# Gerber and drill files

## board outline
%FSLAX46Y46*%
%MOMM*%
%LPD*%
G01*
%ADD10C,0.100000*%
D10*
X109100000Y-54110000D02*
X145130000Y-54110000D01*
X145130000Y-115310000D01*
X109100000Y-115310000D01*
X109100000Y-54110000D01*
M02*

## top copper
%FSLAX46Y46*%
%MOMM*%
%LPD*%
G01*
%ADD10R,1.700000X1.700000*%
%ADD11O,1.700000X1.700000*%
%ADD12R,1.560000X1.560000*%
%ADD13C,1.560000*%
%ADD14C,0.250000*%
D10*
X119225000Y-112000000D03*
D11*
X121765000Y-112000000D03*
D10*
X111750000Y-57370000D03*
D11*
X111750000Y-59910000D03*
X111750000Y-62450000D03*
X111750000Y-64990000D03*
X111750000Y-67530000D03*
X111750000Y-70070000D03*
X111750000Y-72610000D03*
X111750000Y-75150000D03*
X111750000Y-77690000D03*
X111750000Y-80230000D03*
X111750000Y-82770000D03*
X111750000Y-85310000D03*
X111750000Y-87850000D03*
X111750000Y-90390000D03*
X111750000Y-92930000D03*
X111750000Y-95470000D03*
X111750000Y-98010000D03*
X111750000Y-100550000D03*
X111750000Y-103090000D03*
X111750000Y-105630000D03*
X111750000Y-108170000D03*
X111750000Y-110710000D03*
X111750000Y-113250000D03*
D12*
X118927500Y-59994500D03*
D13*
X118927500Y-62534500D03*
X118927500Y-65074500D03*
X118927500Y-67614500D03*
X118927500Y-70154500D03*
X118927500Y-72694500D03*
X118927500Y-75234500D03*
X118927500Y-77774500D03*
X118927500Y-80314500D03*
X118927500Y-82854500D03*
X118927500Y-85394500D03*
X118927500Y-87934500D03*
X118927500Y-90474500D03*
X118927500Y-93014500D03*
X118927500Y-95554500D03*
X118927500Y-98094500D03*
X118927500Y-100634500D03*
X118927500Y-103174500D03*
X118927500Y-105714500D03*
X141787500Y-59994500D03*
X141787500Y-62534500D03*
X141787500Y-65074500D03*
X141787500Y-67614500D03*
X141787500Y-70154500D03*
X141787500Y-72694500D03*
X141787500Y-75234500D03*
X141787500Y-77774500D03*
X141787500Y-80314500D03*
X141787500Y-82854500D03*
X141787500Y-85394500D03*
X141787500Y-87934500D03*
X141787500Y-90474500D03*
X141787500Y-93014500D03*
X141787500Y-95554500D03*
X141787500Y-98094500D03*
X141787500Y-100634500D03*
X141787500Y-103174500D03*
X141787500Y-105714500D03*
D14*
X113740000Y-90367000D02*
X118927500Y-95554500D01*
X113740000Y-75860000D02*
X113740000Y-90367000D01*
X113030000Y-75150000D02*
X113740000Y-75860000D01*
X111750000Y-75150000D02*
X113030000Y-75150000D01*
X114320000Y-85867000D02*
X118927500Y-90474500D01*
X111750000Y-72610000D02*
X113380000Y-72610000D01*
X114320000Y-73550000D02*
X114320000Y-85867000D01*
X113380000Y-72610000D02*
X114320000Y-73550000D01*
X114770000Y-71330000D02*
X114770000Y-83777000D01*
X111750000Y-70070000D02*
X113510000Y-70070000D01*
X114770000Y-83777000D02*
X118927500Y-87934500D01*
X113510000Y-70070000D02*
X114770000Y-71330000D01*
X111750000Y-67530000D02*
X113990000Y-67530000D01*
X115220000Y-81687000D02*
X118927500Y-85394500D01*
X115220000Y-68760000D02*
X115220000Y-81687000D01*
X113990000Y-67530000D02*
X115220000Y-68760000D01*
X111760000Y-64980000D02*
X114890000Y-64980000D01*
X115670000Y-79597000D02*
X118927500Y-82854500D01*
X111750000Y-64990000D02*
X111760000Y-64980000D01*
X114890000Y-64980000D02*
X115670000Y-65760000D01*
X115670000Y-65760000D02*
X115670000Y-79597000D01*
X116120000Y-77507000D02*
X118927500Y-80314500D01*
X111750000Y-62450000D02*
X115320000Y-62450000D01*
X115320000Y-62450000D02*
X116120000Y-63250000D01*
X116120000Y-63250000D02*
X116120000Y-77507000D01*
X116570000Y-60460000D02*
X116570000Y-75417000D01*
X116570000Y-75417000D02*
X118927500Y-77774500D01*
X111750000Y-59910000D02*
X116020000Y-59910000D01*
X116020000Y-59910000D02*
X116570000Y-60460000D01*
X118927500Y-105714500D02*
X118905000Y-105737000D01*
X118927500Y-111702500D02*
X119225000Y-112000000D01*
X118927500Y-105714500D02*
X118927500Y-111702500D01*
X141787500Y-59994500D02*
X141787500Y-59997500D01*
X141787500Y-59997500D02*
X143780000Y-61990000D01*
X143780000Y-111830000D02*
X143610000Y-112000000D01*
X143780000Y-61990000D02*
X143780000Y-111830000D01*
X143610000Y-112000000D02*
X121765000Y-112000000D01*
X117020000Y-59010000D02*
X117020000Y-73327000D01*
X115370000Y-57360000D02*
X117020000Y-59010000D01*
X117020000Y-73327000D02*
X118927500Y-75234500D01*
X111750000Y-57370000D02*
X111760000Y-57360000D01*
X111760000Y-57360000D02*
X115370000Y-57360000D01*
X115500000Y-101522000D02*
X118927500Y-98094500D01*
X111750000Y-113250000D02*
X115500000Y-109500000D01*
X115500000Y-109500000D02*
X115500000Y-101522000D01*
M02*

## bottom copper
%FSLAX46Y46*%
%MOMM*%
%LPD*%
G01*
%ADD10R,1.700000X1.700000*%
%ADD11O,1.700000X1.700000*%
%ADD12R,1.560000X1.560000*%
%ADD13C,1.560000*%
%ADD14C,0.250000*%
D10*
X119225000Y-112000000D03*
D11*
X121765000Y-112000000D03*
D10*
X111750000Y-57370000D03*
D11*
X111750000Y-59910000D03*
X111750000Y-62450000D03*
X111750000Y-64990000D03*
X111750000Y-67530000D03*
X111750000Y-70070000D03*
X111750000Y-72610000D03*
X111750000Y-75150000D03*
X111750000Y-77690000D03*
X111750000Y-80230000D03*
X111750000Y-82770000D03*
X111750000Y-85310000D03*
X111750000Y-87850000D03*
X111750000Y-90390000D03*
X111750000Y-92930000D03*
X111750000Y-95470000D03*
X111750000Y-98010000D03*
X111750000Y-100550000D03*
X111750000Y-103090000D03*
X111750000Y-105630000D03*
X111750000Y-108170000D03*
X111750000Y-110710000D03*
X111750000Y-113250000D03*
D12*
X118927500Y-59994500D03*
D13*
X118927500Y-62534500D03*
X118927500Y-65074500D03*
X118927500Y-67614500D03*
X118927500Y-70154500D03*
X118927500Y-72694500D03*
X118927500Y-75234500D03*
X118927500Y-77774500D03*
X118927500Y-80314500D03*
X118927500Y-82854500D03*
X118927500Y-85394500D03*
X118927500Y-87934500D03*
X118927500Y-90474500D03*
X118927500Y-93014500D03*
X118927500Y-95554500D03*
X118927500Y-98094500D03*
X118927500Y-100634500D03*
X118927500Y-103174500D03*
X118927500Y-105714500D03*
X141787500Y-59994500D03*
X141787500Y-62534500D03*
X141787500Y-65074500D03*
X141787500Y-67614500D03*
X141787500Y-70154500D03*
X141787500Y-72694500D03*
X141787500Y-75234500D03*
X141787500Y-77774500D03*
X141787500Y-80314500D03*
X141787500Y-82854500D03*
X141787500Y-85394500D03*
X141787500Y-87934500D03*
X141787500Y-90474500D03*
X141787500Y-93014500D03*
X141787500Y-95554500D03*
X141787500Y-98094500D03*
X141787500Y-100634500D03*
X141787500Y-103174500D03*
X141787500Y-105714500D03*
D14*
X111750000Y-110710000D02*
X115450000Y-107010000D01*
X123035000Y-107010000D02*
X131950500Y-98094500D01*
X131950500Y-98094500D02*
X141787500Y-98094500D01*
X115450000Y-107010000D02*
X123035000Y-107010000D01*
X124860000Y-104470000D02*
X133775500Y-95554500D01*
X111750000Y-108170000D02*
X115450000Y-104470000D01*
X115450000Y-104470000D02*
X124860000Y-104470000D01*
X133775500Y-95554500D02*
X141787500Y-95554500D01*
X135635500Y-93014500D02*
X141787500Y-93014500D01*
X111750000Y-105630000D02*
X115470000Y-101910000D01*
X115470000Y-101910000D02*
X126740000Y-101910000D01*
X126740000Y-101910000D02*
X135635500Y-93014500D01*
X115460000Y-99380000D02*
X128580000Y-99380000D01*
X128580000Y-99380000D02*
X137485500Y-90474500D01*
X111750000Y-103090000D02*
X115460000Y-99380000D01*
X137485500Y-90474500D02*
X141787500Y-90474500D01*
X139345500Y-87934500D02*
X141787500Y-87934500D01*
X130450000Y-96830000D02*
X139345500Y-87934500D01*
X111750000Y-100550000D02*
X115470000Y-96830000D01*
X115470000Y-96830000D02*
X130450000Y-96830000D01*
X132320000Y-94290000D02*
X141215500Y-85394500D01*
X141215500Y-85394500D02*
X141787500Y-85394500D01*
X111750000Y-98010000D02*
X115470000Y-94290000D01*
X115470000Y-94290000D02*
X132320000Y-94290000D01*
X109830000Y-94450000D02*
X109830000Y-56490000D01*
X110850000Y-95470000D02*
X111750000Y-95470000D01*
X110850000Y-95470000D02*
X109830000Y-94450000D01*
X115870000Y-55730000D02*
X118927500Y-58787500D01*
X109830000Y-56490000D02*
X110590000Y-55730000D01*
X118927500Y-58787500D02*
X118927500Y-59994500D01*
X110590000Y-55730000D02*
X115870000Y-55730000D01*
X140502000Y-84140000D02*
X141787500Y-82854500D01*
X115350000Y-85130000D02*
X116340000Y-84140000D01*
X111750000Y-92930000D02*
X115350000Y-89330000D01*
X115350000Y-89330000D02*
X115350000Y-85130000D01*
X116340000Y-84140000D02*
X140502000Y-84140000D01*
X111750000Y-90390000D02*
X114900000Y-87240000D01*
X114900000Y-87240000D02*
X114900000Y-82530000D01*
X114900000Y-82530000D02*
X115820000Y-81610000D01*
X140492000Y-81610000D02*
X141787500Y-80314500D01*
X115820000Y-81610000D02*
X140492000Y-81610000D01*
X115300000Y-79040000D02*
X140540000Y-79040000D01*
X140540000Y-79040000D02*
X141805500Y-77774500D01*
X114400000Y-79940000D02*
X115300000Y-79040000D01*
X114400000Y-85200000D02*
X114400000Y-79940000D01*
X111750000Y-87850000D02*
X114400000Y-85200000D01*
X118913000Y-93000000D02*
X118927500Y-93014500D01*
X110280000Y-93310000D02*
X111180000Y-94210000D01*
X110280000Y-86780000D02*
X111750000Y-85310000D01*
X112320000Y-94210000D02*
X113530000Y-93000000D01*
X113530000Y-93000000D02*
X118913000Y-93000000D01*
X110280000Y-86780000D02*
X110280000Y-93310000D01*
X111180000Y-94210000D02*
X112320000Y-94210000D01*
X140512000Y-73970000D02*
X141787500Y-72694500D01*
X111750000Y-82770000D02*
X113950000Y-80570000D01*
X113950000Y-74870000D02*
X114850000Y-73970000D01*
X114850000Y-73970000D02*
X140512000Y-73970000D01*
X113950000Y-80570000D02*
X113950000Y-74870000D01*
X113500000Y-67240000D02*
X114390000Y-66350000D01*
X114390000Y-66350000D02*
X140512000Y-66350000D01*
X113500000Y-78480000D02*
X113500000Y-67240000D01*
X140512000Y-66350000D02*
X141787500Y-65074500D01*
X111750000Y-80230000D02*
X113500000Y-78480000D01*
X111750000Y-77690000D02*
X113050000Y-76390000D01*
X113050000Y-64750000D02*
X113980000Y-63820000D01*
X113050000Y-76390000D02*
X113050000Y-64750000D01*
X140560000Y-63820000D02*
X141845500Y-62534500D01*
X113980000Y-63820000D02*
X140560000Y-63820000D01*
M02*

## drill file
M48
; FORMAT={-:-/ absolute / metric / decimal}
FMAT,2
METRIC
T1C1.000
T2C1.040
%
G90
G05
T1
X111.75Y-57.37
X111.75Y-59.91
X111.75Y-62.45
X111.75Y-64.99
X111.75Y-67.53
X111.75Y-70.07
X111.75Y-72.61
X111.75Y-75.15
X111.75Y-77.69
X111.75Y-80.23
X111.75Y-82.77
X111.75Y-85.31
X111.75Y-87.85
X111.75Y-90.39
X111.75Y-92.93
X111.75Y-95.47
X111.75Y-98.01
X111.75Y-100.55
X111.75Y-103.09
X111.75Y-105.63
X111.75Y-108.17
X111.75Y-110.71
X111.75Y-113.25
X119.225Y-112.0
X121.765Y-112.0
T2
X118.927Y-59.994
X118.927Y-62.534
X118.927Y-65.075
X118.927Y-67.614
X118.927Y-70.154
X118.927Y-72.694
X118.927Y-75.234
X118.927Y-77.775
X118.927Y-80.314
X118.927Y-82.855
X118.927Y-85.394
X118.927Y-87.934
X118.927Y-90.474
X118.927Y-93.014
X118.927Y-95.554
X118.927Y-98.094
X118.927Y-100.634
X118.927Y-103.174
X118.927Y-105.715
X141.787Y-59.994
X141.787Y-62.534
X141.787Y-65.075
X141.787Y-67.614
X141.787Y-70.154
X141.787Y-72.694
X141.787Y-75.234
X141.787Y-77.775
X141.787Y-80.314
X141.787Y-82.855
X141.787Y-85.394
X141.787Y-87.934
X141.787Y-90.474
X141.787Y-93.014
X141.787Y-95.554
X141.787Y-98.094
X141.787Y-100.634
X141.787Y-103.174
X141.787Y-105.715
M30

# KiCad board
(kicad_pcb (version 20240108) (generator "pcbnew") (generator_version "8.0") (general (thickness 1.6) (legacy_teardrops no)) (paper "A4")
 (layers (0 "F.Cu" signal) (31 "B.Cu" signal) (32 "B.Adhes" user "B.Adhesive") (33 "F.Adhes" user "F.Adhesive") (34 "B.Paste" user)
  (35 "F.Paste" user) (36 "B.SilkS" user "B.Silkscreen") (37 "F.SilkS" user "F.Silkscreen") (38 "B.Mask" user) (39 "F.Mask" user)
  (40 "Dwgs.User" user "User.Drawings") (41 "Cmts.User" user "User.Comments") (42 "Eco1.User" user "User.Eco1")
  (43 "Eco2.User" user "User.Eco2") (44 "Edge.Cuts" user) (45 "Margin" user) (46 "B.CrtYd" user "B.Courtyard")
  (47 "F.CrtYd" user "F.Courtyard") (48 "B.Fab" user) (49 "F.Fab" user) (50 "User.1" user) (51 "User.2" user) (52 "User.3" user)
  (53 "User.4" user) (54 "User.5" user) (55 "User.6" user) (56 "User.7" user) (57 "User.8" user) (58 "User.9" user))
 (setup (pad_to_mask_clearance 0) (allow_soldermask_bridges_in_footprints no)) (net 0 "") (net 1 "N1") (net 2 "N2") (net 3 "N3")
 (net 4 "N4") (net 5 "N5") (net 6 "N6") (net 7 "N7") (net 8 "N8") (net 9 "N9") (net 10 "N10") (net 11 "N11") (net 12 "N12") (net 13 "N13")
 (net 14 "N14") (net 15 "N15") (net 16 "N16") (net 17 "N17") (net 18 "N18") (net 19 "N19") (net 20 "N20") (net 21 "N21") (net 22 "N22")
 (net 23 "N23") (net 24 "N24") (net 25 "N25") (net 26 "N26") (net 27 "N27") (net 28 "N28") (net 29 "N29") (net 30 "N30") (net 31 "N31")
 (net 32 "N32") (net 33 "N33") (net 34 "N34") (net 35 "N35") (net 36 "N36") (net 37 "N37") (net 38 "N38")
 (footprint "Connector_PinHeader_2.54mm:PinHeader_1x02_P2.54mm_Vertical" (layer "F.Cu") (at 119.225 112 90)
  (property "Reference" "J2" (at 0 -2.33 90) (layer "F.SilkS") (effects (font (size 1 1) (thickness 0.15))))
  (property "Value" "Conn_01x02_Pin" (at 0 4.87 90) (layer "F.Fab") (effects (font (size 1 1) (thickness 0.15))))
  (pad "1" thru_hole rect (at 0 0 90) (size 1.7 1.7) (drill 1) (layers "*.Cu" "*.Mask") (remove_unused_layers no) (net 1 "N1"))
  (pad "2" thru_hole oval (at 0 2.54 90) (size 1.7 1.7) (drill 1) (layers "*.Cu" "*.Mask") (remove_unused_layers no) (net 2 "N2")))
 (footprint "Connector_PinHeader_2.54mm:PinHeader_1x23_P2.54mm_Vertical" (layer "F.Cu") (at 111.75 57.37)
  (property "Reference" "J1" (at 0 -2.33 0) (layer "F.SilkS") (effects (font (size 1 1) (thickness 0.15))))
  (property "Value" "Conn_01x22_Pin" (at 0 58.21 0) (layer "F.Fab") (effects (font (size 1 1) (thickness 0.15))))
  (pad "1" thru_hole rect (at 0 0) (size 1.7 1.7) (drill 1) (layers "*.Cu" "*.Mask") (remove_unused_layers no) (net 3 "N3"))
  (pad "2" thru_hole oval (at 0 2.54) (size 1.7 1.7) (drill 1) (layers "*.Cu" "*.Mask") (remove_unused_layers no) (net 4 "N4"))
  (pad "3" thru_hole oval (at 0 5.08) (size 1.7 1.7) (drill 1) (layers "*.Cu" "*.Mask") (remove_unused_layers no) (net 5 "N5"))
  (pad "4" thru_hole oval (at 0 7.62) (size 1.7 1.7) (drill 1) (layers "*.Cu" "*.Mask") (remove_unused_layers no) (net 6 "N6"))
  (pad "5" thru_hole oval (at 0 10.16) (size 1.7 1.7) (drill 1) (layers "*.Cu" "*.Mask") (remove_unused_layers no) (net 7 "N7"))
  (pad "6" thru_hole oval (at 0 12.7) (size 1.7 1.7) (drill 1) (layers "*.Cu" "*.Mask") (remove_unused_layers no) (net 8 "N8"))
  (pad "7" thru_hole oval (at 0 15.24) (size 1.7 1.7) (drill 1) (layers "*.Cu" "*.Mask") (remove_unused_layers no) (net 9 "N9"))
  (pad "8" thru_hole oval (at 0 17.78) (size 1.7 1.7) (drill 1) (layers "*.Cu" "*.Mask") (remove_unused_layers no) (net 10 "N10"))
  (pad "9" thru_hole oval (at 0 20.32) (size 1.7 1.7) (drill 1) (layers "*.Cu" "*.Mask") (remove_unused_layers no) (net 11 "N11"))
  (pad "10" thru_hole oval (at 0 22.86) (size 1.7 1.7) (drill 1) (layers "*.Cu" "*.Mask") (remove_unused_layers no) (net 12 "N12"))
  (pad "11" thru_hole oval (at 0 25.4) (size 1.7 1.7) (drill 1) (layers "*.Cu" "*.Mask") (remove_unused_layers no) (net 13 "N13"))
  (pad "12" thru_hole oval (at 0 27.94) (size 1.7 1.7) (drill 1) (layers "*.Cu" "*.Mask") (remove_unused_layers no) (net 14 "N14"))
  (pad "13" thru_hole oval (at 0 30.48) (size 1.7 1.7) (drill 1) (layers "*.Cu" "*.Mask") (remove_unused_layers no) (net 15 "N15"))
  (pad "14" thru_hole oval (at 0 33.02) (size 1.7 1.7) (drill 1) (layers "*.Cu" "*.Mask") (remove_unused_layers no) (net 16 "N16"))
  (pad "15" thru_hole oval (at 0 35.56) (size 1.7 1.7) (drill 1) (layers "*.Cu" "*.Mask") (remove_unused_layers no) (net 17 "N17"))
  (pad "16" thru_hole oval (at 0 38.1) (size 1.7 1.7) (drill 1) (layers "*.Cu" "*.Mask") (remove_unused_layers no) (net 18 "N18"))
  (pad "17" thru_hole oval (at 0 40.64) (size 1.7 1.7) (drill 1) (layers "*.Cu" "*.Mask") (remove_unused_layers no) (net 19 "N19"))
  (pad "18" thru_hole oval (at 0 43.18) (size 1.7 1.7) (drill 1) (layers "*.Cu" "*.Mask") (remove_unused_layers no) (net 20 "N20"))
  (pad "19" thru_hole oval (at 0 45.72) (size 1.7 1.7) (drill 1) (layers "*.Cu" "*.Mask") (remove_unused_layers no) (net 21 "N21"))
  (pad "20" thru_hole oval (at 0 48.26) (size 1.7 1.7) (drill 1) (layers "*.Cu" "*.Mask") (remove_unused_layers no) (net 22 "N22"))
  (pad "21" thru_hole oval (at 0 50.8) (size 1.7 1.7) (drill 1) (layers "*.Cu" "*.Mask") (remove_unused_layers no) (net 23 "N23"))
  (pad "22" thru_hole oval (at 0 53.34) (size 1.7 1.7) (drill 1) (layers "*.Cu" "*.Mask") (remove_unused_layers no) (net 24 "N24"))
  (pad "23" thru_hole oval (at 0 55.88) (size 1.7 1.7) (drill 1) (layers "*.Cu" "*.Mask") (remove_unused_layers no) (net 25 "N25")))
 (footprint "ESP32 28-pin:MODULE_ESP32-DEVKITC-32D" (layer "F.Cu") (at 131.6275 79.7545)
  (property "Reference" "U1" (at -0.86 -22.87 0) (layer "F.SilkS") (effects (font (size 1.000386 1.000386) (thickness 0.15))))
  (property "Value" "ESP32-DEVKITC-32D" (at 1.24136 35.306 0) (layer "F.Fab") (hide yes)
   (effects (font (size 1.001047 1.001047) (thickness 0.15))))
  (pad "J2-1" thru_hole rect (at -12.7 -19.76) (size 1.56 1.56) (drill 1.04) (layers "*.Cu" "*.Mask") (remove_unused_layers no)
   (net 18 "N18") (solder_mask_margin 0.102))
  (pad "J2-2" thru_hole circle (at -12.7 -17.22) (size 1.56 1.56) (drill 1.04) (layers "*.Cu" "*.Mask") (remove_unused_layers no)
   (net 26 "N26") (solder_mask_margin 0.102))
  (pad "J2-3" thru_hole circle (at -12.7 -14.68) (size 1.56 1.56) (drill 1.04) (layers "*.Cu" "*.Mask") (remove_unused_layers no)
   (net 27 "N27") (solder_mask_margin 0.102))
  (pad "J2-4" thru_hole circle (at -12.7 -12.14) (size 1.56 1.56) (drill 1.04) (layers "*.Cu" "*.Mask") (remove_unused_layers no)
   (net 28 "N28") (solder_mask_margin 0.102))
  (pad "J2-5" thru_hole circle (at -12.7 -9.6) (size 1.56 1.56) (drill 1.04) (layers "*.Cu" "*.Mask") (remove_unused_layers no)
   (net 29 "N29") (solder_mask_margin 0.102))
  (pad "J2-6" thru_hole circle (at -12.7 -7.06) (size 1.56 1.56) (drill 1.04) (layers "*.Cu" "*.Mask") (remove_unused_layers no)
   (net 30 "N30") (solder_mask_margin 0.102))
  (pad "J2-7" thru_hole circle (at -12.7 -4.52) (size 1.56 1.56) (drill 1.04) (layers "*.Cu" "*.Mask") (remove_unused_layers no)
   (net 3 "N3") (solder_mask_margin 0.102))
  (pad "J2-8" thru_hole circle (at -12.7 -1.98) (size 1.56 1.56) (drill 1.04) (layers "*.Cu" "*.Mask") (remove_unused_layers no)
   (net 4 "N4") (solder_mask_margin 0.102))
  (pad "J2-9" thru_hole circle (at -12.7 0.56) (size 1.56 1.56) (drill 1.04) (layers "*.Cu" "*.Mask") (remove_unused_layers no) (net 5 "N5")
   (solder_mask_margin 0.102))
  (pad "J2-10" thru_hole circle (at -12.7 3.1) (size 1.56 1.56) (drill 1.04) (layers "*.Cu" "*.Mask") (remove_unused_layers no) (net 6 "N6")
   (solder_mask_margin 0.102))
  (pad "J2-11" thru_hole circle (at -12.7 5.64) (size 1.56 1.56) (drill 1.04) (layers "*.Cu" "*.Mask") (remove_unused_layers no)
   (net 7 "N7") (solder_mask_margin 0.102))
  (pad "J2-12" thru_hole circle (at -12.7 8.18) (size 1.56 1.56) (drill 1.04) (layers "*.Cu" "*.Mask") (remove_unused_layers no)
   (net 8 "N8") (solder_mask_margin 0.102))
  (pad "J2-13" thru_hole circle (at -12.7 10.72) (size 1.56 1.56) (drill 1.04) (layers "*.Cu" "*.Mask") (remove_unused_layers no)
   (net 9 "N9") (solder_mask_margin 0.102))
  (pad "J2-14" thru_hole circle (at -12.7 13.26) (size 1.56 1.56) (drill 1.04) (layers "*.Cu" "*.Mask") (remove_unused_layers no)
   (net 14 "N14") (solder_mask_margin 0.102))
  (pad "J2-15" thru_hole circle (at -12.7 15.8) (size 1.56 1.56) (drill 1.04) (layers "*.Cu" "*.Mask") (remove_unused_layers no)
   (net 10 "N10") (solder_mask_margin 0.102))
  (pad "J2-16" thru_hole circle (at -12.7 18.34) (size 1.56 1.56) (drill 1.04) (layers "*.Cu" "*.Mask") (remove_unused_layers no)
   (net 25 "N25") (solder_mask_margin 0.102))
  (pad "J2-17" thru_hole circle (at -12.7 20.88) (size 1.56 1.56) (drill 1.04) (layers "*.Cu" "*.Mask") (remove_unused_layers no)
   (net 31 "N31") (solder_mask_margin 0.102))
  (pad "J2-18" thru_hole circle (at -12.7 23.42) (size 1.56 1.56) (drill 1.04) (layers "*.Cu" "*.Mask") (remove_unused_layers no)
   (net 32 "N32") (solder_mask_margin 0.102))
  (pad "J2-19" thru_hole circle (at -12.7 25.96) (size 1.56 1.56) (drill 1.04) (layers "*.Cu" "*.Mask") (remove_unused_layers no)
   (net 1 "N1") (solder_mask_margin 0.102))
  (pad "J3-1" thru_hole circle (at 10.16 -19.76) (size 1.56 1.56) (drill 1.04) (layers "*.Cu" "*.Mask") (remove_unused_layers no)
   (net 2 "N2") (solder_mask_margin 0.102))
  (pad "J3-2" thru_hole circle (at 10.16 -17.22) (size 1.56 1.56) (drill 1.04) (layers "*.Cu" "*.Mask") (remove_unused_layers no)
   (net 11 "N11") (solder_mask_margin 0.102))
  (pad "J3-3" thru_hole circle (at 10.16 -14.68) (size 1.56 1.56) (drill 1.04) (layers "*.Cu" "*.Mask") (remove_unused_layers no)
   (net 12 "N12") (solder_mask_margin 0.102))
  (pad "J3-4" thru_hole circle (at 10.16 -12.14) (size 1.56 1.56) (drill 1.04) (layers "*.Cu" "*.Mask") (remove_unused_layers no)
   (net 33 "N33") (solder_mask_margin 0.102))
  (pad "J3-5" thru_hole circle (at 10.16 -9.6) (size 1.56 1.56) (drill 1.04) (layers "*.Cu" "*.Mask") (remove_unused_layers no)
   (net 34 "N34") (solder_mask_margin 0.102))
  (pad "J3-6" thru_hole circle (at 10.16 -7.06) (size 1.56 1.56) (drill 1.04) (layers "*.Cu" "*.Mask") (remove_unused_layers no)
   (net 13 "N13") (solder_mask_margin 0.102))
  (pad "J3-7" thru_hole circle (at 10.16 -4.52) (size 1.56 1.56) (drill 1.04) (layers "*.Cu" "*.Mask") (remove_unused_layers no)
   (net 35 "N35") (solder_mask_margin 0.102))
  (pad "J3-8" thru_hole circle (at 10.16 -1.98) (size 1.56 1.56) (drill 1.04) (layers "*.Cu" "*.Mask") (remove_unused_layers no)
   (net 15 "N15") (solder_mask_margin 0.102))
  (pad "J3-9" thru_hole circle (at 10.16 0.56) (size 1.56 1.56) (drill 1.04) (layers "*.Cu" "*.Mask") (remove_unused_layers no)
   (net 16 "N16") (solder_mask_margin 0.102))
  (pad "J3-10" thru_hole circle (at 10.16 3.1) (size 1.56 1.56) (drill 1.04) (layers "*.Cu" "*.Mask") (remove_unused_layers no)
   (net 17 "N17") (solder_mask_margin 0.102))
  (pad "J3-11" thru_hole circle (at 10.16 5.64) (size 1.56 1.56) (drill 1.04) (layers "*.Cu" "*.Mask") (remove_unused_layers no)
   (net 19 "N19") (solder_mask_margin 0.102))
  (pad "J3-12" thru_hole circle (at 10.16 8.18) (size 1.56 1.56) (drill 1.04) (layers "*.Cu" "*.Mask") (remove_unused_layers no)
   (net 20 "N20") (solder_mask_margin 0.102))
  (pad "J3-13" thru_hole circle (at 10.16 10.72) (size 1.56 1.56) (drill 1.04) (layers "*.Cu" "*.Mask") (remove_unused_layers no)
   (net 21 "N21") (solder_mask_margin 0.102))
  (pad "J3-14" thru_hole circle (at 10.16 13.26) (size 1.56 1.56) (drill 1.04) (layers "*.Cu" "*.Mask") (remove_unused_layers no)
   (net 22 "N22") (solder_mask_margin 0.102))
  (pad "J3-15" thru_hole circle (at 10.16 15.8) (size 1.56 1.56) (drill 1.04) (layers "*.Cu" "*.Mask") (remove_unused_layers no)
   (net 23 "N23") (solder_mask_margin 0.102))
  (pad "J3-16" thru_hole circle (at 10.16 18.34) (size 1.56 1.56) (drill 1.04) (layers "*.Cu" "*.Mask") (remove_unused_layers no)
   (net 24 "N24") (solder_mask_margin 0.102))
  (pad "J3-17" thru_hole circle (at 10.16 20.88) (size 1.56 1.56) (drill 1.04) (layers "*.Cu" "*.Mask") (remove_unused_layers no)
   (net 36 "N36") (solder_mask_margin 0.102))
  (pad "J3-18" thru_hole circle (at 10.16 23.42) (size 1.56 1.56) (drill 1.04) (layers "*.Cu" "*.Mask") (remove_unused_layers no)
   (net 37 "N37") (solder_mask_margin 0.102))
  (pad "J3-19" thru_hole circle (at 10.16 25.96) (size 1.56 1.56) (drill 1.04) (layers "*.Cu" "*.Mask") (remove_unused_layers no)
   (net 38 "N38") (solder_mask_margin 0.102)))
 (gr_rect (start 109.1 54.11) (end 145.13 115.31) (stroke (width 0.1) (type default)) (fill none) (layer "Edge.Cuts"))
 (segment (start 111.75 110.71) (end 115.45 107.01) (width 0.25) (layer "B.Cu") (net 24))
 (segment (start 123.035 107.01) (end 131.9505 98.0945) (width 0.25) (layer "B.Cu") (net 24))
 (segment (start 131.9505 98.0945) (end 141.7875 98.0945) (width 0.25) (layer "B.Cu") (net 24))
 (segment (start 115.45 107.01) (end 123.035 107.01) (width 0.25) (layer "B.Cu") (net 24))
 (segment (start 124.86 104.47) (end 133.7755 95.5545) (width 0.25) (layer "B.Cu") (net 23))
 (segment (start 111.75 108.17) (end 115.45 104.47) (width 0.25) (layer "B.Cu") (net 23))
 (segment (start 115.45 104.47) (end 124.86 104.47) (width 0.25) (layer "B.Cu") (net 23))
 (segment (start 133.7755 95.5545) (end 141.7875 95.5545) (width 0.25) (layer "B.Cu") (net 23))
 (segment (start 135.6355 93.0145) (end 141.7875 93.0145) (width 0.25) (layer "B.Cu") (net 22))
 (segment (start 111.75 105.63) (end 115.47 101.91) (width 0.25) (layer "B.Cu") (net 22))
 (segment (start 115.47 101.91) (end 126.74 101.91) (width 0.25) (layer "B.Cu") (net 22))
 (segment (start 126.74 101.91) (end 135.6355 93.0145) (width 0.25) (layer "B.Cu") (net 22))
 (segment (start 115.46 99.38) (end 128.58 99.38) (width 0.25) (layer "B.Cu") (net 21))
 (segment (start 128.58 99.38) (end 137.4855 90.4745) (width 0.25) (layer "B.Cu") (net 21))
 (segment (start 111.75 103.09) (end 115.46 99.38) (width 0.25) (layer "B.Cu") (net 21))
 (segment (start 137.4855 90.4745) (end 141.7875 90.4745) (width 0.25) (layer "B.Cu") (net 21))
 (segment (start 139.3455 87.9345) (end 141.7875 87.9345) (width 0.25) (layer "B.Cu") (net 20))
 (segment (start 130.45 96.83) (end 139.3455 87.9345) (width 0.25) (layer "B.Cu") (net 20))
 (segment (start 111.75 100.55) (end 115.47 96.83) (width 0.25) (layer "B.Cu") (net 20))
 (segment (start 115.47 96.83) (end 130.45 96.83) (width 0.25) (layer "B.Cu") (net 20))
 (segment (start 132.32 94.29) (end 141.2155 85.3945) (width 0.25) (layer "B.Cu") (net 19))
 (segment (start 141.2155 85.3945) (end 141.7875 85.3945) (width 0.25) (layer "B.Cu") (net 19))
 (segment (start 111.75 98.01) (end 115.47 94.29) (width 0.25) (layer "B.Cu") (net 19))
 (segment (start 115.47 94.29) (end 132.32 94.29) (width 0.25) (layer "B.Cu") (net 19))
 (segment (start 109.83 94.45) (end 109.83 56.49) (width 0.25) (layer "B.Cu") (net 18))
 (segment (start 110.85 95.47) (end 111.75 95.47) (width 0.25) (layer "B.Cu") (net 18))
 (segment (start 110.85 95.47) (end 109.83 94.45) (width 0.25) (layer "B.Cu") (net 18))
 (segment (start 115.87 55.73) (end 118.9275 58.7875) (width 0.25) (layer "B.Cu") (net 18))
 (segment (start 109.83 56.49) (end 110.59 55.73) (width 0.25) (layer "B.Cu") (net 18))
 (segment (start 118.9275 58.7875) (end 118.9275 59.9945) (width 0.25) (layer "B.Cu") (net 18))
 (segment (start 110.59 55.73) (end 115.87 55.73) (width 0.25) (layer "B.Cu") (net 18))
 (segment (start 140.502 84.14) (end 141.7875 82.8545) (width 0.25) (layer "B.Cu") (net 17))
 (segment (start 115.35 85.13) (end 116.34 84.14) (width 0.25) (layer "B.Cu") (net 17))
 (segment (start 111.75 92.93) (end 115.35 89.33) (width 0.25) (layer "B.Cu") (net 17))
 (segment (start 115.35 89.33) (end 115.35 85.13) (width 0.25) (layer "B.Cu") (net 17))
 (segment (start 116.34 84.14) (end 140.502 84.14) (width 0.25) (layer "B.Cu") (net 17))
 (segment (start 111.75 90.39) (end 114.9 87.24) (width 0.25) (layer "B.Cu") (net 16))
 (segment (start 114.9 87.24) (end 114.9 82.53) (width 0.25) (layer "B.Cu") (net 16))
 (segment (start 114.9 82.53) (end 115.82 81.61) (width 0.25) (layer "B.Cu") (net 16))
 (segment (start 140.492 81.61) (end 141.7875 80.3145) (width 0.25) (layer "B.Cu") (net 16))
 (segment (start 115.82 81.61) (end 140.492 81.61) (width 0.25) (layer "B.Cu") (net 16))
 (segment (start 115.3 79.04) (end 140.54 79.04) (width 0.25) (layer "B.Cu") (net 15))
 (segment (start 140.54 79.04) (end 141.8055 77.7745) (width 0.25) (layer "B.Cu") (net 15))
 (segment (start 114.4 79.94) (end 115.3 79.04) (width 0.25) (layer "B.Cu") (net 15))
 (segment (start 114.4 85.2) (end 114.4 79.94) (width 0.25) (layer "B.Cu") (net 15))
 (segment (start 111.75 87.85) (end 114.4 85.2) (width 0.25) (layer "B.Cu") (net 15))
 (segment (start 118.913 93) (end 118.9275 93.0145) (width 0.25) (layer "B.Cu") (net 14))
 (segment (start 110.28 93.31) (end 111.18 94.21) (width 0.25) (layer "B.Cu") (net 14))
 (segment (start 110.28 86.78) (end 111.75 85.31) (width 0.25) (layer "B.Cu") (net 14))
 (segment (start 112.32 94.21) (end 113.53 93) (width 0.25) (layer "B.Cu") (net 14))
 (segment (start 113.53 93) (end 118.913 93) (width 0.25) (layer "B.Cu") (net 14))
 (segment (start 110.28 86.78) (end 110.28 93.31) (width 0.25) (layer "B.Cu") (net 14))
 (segment (start 111.18 94.21) (end 112.32 94.21) (width 0.25) (layer "B.Cu") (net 14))
 (segment (start 140.512 73.97) (end 141.7875 72.6945) (width 0.25) (layer "B.Cu") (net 13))
 (segment (start 111.75 82.77) (end 113.95 80.57) (width 0.25) (layer "B.Cu") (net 13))
 (segment (start 113.95 74.87) (end 114.85 73.97) (width 0.25) (layer "B.Cu") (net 13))
 (segment (start 114.85 73.97) (end 140.512 73.97) (width 0.25) (layer "B.Cu") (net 13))
 (segment (start 113.95 80.57) (end 113.95 74.87) (width 0.25) (layer "B.Cu") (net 13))
 (segment (start 113.5 67.24) (end 114.39 66.35) (width 0.25) (layer "B.Cu") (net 12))
 (segment (start 114.39 66.35) (end 140.512 66.35) (width 0.25) (layer "B.Cu") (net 12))
 (segment (start 113.5 78.48) (end 113.5 67.24) (width 0.25) (layer "B.Cu") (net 12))
 (segment (start 140.512 66.35) (end 141.7875 65.0745) (width 0.25) (layer "B.Cu") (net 12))
 (segment (start 111.75 80.23) (end 113.5 78.48) (width 0.25) (layer "B.Cu") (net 12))
 (segment (start 111.75 77.69) (end 113.05 76.39) (width 0.25) (layer "B.Cu") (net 11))
 (segment (start 113.05 64.75) (end 113.98 63.82) (width 0.25) (layer "B.Cu") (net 11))
 (segment (start 113.05 76.39) (end 113.05 64.75) (width 0.25) (layer "B.Cu") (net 11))
 (segment (start 140.56 63.82) (end 141.8455 62.5345) (width 0.25) (layer "B.Cu") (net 11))
 (segment (start 113.98 63.82) (end 140.56 63.82) (width 0.25) (layer "B.Cu") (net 11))
 (segment (start 113.74 90.367) (end 118.9275 95.5545) (width 0.25) (layer "F.Cu") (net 10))
 (segment (start 113.74 75.86) (end 113.74 90.367) (width 0.25) (layer "F.Cu") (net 10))
 (segment (start 113.03 75.15) (end 113.74 75.86) (width 0.25) (layer "F.Cu") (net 10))
 (segment (start 111.75 75.15) (end 113.03 75.15) (width 0.25) (layer "F.Cu") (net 10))
 (segment (start 114.32 85.867) (end 118.9275 90.4745) (width 0.25) (layer "F.Cu") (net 9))
 (segment (start 111.75 72.61) (end 113.38 72.61) (width 0.25) (layer "F.Cu") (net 9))
 (segment (start 114.32 73.55) (end 114.32 85.867) (width 0.25) (layer "F.Cu") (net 9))
 (segment (start 113.38 72.61) (end 114.32 73.55) (width 0.25) (layer "F.Cu") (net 9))
 (segment (start 114.77 71.33) (end 114.77 83.777) (width 0.25) (layer "F.Cu") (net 8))
 (segment (start 111.75 70.07) (end 113.51 70.07) (width 0.25) (layer "F.Cu") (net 8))
 (segment (start 114.77 83.777) (end 118.9275 87.9345) (width 0.25) (layer "F.Cu") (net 8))
 (segment (start 113.51 70.07) (end 114.77 71.33) (width 0.25) (layer "F.Cu") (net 8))
 (segment (start 111.75 67.53) (end 113.99 67.53) (width 0.25) (layer "F.Cu") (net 7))
 (segment (start 115.22 81.687) (end 118.9275 85.3945) (width 0.25) (layer "F.Cu") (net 7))
 (segment (start 115.22 68.76) (end 115.22 81.687) (width 0.25) (layer "F.Cu") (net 7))
 (segment (start 113.99 67.53) (end 115.22 68.76) (width 0.25) (layer "F.Cu") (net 7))
 (segment (start 111.76 64.98) (end 114.89 64.98) (width 0.25) (layer "F.Cu") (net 6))
 (segment (start 115.67 79.597) (end 118.9275 82.8545) (width 0.25) (layer "F.Cu") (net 6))
 (segment (start 111.75 64.99) (end 111.76 64.98) (width 0.25) (layer "F.Cu") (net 6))
 (segment (start 114.89 64.98) (end 115.67 65.76) (width 0.25) (layer "F.Cu") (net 6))
 (segment (start 115.67 65.76) (end 115.67 79.597) (width 0.25) (layer "F.Cu") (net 6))
 (segment (start 116.12 77.507) (end 118.9275 80.3145) (width 0.25) (layer "F.Cu") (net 5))
 (segment (start 111.75 62.45) (end 115.32 62.45) (width 0.25) (layer "F.Cu") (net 5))
 (segment (start 115.32 62.45) (end 116.12 63.25) (width 0.25) (layer "F.Cu") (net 5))
 (segment (start 116.12 63.25) (end 116.12 77.507) (width 0.25) (layer "F.Cu") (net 5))
 (segment (start 116.57 60.46) (end 116.57 75.417) (width 0.25) (layer "F.Cu") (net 4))
 (segment (start 116.57 75.417) (end 118.9275 77.7745) (width 0.25) (layer "F.Cu") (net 4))
 (segment (start 111.75 59.91) (end 116.02 59.91) (width 0.25) (layer "F.Cu") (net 4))
 (segment (start 116.02 59.91) (end 116.57 60.46) (width 0.25) (layer "F.Cu") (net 4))
 (segment (start 118.9275 105.7145) (end 118.905 105.737) (width 0.25) (layer "F.Cu") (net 1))
 (segment (start 118.9275 111.7025) (end 119.225 112) (width 0.25) (layer "F.Cu") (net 1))
 (segment (start 118.9275 105.7145) (end 118.9275 111.7025) (width 0.25) (layer "F.Cu") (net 1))
 (segment (start 141.7875 59.9945) (end 141.7875 59.9975) (width 0.25) (layer "F.Cu") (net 2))
 (segment (start 141.7875 59.9975) (end 143.78 61.99) (width 0.25) (layer "F.Cu") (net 2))
 (segment (start 143.78 111.83) (end 143.61 112) (width 0.25) (layer "F.Cu") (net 2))
 (segment (start 143.78 61.99) (end 143.78 111.83) (width 0.25) (layer "F.Cu") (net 2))
 (segment (start 143.61 112) (end 121.765 112) (width 0.25) (layer "F.Cu") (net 2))
 (segment (start 117.02 59.01) (end 117.02 73.327) (width 0.25) (layer "F.Cu") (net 3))
 (segment (start 115.37 57.36) (end 117.02 59.01) (width 0.25) (layer "F.Cu") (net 3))
 (segment (start 117.02 73.327) (end 118.9275 75.2345) (width 0.25) (layer "F.Cu") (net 3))
 (segment (start 111.75 57.37) (end 111.76 57.36) (width 0.25) (layer "F.Cu") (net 3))
 (segment (start 111.76 57.36) (end 115.37 57.36) (width 0.25) (layer "F.Cu") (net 3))
 (segment (start 115.5 101.522) (end 118.9275 98.0945) (width 0.25) (layer "F.Cu") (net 25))
 (segment (start 111.75 113.25) (end 115.5 109.5) (width 0.25) (layer "F.Cu") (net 25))
 (segment (start 115.5 109.5) (end 115.5 101.522) (width 0.25) (layer "F.Cu") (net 25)))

